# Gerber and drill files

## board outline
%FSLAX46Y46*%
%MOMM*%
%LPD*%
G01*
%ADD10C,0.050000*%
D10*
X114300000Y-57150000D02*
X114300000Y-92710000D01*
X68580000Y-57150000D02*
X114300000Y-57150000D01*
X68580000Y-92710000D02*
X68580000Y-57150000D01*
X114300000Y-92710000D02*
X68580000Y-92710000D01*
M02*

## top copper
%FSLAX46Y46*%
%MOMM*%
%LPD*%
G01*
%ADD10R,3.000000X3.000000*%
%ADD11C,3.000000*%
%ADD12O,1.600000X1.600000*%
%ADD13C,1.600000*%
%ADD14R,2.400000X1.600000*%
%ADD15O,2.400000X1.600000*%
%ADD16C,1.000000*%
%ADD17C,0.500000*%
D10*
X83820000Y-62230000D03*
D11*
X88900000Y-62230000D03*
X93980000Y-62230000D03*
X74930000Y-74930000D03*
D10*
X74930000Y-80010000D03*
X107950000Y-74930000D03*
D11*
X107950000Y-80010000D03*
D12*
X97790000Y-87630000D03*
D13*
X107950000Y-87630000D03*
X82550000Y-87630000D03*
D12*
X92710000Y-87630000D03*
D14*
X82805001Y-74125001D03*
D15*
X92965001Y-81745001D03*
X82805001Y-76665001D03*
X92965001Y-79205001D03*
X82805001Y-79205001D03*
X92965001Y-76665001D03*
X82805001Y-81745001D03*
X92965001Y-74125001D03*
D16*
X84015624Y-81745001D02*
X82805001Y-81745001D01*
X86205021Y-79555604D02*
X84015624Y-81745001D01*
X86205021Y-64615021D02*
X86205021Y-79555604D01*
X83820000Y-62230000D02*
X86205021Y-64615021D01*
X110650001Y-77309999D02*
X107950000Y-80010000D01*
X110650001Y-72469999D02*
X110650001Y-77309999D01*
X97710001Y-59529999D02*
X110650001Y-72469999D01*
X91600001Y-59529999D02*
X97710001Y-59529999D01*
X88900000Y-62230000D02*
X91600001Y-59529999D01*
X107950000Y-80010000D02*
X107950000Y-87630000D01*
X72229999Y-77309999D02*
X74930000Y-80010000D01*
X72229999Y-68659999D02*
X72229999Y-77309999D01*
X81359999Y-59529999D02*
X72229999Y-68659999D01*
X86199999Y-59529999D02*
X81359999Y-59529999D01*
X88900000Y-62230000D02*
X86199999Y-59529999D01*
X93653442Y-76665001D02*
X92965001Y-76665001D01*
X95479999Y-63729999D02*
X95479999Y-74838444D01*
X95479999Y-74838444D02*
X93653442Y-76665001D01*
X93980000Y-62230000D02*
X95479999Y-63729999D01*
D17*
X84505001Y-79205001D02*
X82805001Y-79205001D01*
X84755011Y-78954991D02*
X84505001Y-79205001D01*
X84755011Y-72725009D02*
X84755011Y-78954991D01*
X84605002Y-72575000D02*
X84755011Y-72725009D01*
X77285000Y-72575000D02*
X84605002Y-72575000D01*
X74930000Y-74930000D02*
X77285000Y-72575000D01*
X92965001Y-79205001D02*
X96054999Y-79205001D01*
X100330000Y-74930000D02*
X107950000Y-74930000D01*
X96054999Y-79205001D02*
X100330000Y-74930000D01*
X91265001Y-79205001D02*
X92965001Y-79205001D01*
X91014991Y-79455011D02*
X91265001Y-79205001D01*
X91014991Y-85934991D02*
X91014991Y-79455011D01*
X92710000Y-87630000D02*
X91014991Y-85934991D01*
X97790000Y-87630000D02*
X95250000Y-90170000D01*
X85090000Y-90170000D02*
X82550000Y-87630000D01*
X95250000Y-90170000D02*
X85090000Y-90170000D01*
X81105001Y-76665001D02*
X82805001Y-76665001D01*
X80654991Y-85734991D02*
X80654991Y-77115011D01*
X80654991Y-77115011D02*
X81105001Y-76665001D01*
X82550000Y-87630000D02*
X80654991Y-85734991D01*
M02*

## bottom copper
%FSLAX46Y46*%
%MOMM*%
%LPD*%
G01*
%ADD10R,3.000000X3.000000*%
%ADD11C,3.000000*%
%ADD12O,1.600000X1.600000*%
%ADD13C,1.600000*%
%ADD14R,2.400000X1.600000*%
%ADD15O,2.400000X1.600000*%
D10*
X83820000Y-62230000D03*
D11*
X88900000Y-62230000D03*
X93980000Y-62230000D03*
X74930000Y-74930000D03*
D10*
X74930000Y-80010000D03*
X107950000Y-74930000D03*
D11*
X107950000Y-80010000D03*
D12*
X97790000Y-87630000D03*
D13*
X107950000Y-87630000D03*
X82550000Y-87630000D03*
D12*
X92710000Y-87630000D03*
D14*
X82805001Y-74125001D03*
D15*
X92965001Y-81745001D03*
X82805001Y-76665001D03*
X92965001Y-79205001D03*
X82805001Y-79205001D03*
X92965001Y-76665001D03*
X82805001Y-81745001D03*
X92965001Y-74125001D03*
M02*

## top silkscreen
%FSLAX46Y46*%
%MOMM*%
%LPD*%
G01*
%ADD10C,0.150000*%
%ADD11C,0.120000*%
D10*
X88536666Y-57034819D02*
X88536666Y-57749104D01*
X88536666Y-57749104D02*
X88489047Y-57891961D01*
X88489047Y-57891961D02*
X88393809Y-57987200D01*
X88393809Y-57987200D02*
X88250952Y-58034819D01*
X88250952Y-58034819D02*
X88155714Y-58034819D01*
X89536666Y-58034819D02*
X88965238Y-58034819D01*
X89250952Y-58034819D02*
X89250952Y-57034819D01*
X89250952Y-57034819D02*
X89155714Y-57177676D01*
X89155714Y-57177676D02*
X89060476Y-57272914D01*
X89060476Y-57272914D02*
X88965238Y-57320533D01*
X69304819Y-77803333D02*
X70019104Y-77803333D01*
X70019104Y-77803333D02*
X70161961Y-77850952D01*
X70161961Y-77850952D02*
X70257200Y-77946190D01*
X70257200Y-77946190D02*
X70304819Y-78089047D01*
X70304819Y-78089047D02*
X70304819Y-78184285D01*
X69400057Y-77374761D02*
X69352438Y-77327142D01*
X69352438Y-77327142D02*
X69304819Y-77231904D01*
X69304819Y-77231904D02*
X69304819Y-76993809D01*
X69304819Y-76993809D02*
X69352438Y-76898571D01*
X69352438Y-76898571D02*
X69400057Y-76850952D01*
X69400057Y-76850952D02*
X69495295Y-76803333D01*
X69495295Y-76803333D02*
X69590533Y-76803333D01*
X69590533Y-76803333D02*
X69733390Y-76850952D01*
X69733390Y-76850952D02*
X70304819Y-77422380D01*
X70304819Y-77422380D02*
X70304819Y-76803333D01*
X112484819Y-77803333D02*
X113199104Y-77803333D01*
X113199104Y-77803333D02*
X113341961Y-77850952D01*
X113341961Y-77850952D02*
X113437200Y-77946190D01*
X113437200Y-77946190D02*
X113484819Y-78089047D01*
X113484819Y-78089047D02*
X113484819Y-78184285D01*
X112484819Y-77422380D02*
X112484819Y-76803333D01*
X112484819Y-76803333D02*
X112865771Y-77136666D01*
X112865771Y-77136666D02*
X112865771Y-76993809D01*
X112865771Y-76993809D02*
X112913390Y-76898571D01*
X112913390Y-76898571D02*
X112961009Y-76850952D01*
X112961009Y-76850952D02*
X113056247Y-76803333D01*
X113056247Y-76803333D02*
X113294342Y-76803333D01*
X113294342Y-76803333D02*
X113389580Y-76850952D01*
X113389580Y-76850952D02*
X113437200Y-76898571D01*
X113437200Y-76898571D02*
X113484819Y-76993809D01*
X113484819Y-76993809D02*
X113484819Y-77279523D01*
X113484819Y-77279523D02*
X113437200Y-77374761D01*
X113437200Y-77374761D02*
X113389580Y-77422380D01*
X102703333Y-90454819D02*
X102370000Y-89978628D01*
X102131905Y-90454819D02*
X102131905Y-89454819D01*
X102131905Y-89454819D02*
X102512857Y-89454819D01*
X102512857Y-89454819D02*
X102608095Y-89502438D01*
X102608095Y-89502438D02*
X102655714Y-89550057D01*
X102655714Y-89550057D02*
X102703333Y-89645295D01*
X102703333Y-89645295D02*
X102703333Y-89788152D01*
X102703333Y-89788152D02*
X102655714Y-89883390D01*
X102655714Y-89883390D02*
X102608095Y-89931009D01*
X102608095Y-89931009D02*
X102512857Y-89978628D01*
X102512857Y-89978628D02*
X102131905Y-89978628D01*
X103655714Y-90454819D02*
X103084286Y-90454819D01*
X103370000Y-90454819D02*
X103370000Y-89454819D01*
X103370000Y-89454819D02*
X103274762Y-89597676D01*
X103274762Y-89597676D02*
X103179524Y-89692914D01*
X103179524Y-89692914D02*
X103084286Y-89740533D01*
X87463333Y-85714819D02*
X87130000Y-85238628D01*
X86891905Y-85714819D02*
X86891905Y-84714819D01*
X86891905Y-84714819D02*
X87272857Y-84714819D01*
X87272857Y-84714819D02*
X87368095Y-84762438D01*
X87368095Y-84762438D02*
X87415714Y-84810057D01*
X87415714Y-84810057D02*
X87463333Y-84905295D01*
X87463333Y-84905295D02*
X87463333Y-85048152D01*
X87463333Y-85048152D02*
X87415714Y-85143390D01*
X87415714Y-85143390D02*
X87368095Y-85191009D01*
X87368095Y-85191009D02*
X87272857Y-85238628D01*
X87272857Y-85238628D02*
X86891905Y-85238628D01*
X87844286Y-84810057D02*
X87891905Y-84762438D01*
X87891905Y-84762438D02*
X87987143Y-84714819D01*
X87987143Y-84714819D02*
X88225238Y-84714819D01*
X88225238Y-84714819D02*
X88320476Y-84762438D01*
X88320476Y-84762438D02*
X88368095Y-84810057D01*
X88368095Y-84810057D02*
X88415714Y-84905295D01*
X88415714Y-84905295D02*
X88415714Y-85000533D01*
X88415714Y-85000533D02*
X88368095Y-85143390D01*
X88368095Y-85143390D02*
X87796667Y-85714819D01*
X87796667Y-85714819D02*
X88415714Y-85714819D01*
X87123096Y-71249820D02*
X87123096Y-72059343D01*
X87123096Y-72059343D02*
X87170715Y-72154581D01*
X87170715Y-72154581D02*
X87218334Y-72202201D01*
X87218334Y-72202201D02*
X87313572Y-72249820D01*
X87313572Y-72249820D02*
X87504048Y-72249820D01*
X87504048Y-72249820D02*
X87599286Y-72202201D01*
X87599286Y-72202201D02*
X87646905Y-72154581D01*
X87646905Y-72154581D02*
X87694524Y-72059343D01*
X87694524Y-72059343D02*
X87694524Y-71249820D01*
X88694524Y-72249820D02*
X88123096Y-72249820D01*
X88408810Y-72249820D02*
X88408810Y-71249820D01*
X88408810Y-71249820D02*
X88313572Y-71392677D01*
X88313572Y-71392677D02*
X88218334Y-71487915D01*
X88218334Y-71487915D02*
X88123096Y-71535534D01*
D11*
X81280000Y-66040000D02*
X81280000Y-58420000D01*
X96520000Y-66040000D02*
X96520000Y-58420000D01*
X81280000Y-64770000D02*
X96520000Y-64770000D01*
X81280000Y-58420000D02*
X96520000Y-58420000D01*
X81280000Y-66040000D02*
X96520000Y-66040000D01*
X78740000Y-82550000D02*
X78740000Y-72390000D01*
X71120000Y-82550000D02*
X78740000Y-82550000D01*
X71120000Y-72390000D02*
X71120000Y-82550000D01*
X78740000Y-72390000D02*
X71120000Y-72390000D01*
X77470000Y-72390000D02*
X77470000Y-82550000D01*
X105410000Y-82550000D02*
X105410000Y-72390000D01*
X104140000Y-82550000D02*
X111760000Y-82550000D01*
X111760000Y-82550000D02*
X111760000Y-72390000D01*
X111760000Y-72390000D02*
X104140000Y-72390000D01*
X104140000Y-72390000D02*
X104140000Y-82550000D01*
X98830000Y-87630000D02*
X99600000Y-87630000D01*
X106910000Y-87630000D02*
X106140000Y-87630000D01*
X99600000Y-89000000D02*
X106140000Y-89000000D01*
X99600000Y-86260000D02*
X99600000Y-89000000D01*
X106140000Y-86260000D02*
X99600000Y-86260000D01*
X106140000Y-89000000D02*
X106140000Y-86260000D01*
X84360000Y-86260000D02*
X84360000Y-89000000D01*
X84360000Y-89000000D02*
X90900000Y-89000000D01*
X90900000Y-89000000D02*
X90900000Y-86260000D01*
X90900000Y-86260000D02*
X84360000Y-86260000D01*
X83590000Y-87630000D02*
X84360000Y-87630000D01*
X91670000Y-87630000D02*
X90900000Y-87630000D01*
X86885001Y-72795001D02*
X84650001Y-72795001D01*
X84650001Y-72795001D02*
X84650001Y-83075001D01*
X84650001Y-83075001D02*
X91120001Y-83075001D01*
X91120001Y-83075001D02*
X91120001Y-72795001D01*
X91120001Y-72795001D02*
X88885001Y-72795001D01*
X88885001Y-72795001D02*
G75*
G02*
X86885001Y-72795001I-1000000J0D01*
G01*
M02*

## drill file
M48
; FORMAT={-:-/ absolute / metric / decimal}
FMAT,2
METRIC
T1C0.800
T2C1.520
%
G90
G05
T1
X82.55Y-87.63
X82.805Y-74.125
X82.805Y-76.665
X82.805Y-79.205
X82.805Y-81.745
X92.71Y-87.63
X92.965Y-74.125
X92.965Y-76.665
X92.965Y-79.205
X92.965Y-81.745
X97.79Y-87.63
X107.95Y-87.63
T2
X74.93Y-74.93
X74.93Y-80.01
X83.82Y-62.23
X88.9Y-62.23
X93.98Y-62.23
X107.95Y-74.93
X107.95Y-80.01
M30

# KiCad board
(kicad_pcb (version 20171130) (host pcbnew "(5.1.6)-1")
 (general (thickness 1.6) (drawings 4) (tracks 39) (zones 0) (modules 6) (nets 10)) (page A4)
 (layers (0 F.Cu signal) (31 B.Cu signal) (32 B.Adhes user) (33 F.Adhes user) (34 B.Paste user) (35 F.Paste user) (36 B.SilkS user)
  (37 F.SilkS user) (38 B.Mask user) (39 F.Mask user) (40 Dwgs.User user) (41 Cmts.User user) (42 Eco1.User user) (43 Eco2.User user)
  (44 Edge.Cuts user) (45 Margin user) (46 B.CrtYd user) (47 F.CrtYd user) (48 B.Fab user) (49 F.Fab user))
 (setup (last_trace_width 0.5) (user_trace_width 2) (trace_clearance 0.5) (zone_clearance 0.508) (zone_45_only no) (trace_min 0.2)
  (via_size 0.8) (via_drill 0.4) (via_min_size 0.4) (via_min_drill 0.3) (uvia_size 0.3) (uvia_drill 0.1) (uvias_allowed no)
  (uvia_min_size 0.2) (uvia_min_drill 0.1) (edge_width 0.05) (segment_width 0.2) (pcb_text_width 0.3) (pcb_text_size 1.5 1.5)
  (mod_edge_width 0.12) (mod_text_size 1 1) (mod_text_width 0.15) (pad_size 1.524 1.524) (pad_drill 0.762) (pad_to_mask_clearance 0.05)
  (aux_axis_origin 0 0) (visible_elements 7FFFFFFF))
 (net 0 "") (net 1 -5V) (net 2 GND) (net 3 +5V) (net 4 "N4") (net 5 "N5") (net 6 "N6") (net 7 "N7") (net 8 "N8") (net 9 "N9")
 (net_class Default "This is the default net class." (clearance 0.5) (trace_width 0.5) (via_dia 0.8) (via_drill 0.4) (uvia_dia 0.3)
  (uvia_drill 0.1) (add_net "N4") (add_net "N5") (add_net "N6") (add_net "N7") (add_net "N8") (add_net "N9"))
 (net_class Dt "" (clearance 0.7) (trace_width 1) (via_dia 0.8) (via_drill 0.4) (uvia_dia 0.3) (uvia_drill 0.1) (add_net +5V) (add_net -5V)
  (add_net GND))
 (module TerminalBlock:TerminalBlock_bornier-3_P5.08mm (layer F.Cu) (at 83.82 62.23)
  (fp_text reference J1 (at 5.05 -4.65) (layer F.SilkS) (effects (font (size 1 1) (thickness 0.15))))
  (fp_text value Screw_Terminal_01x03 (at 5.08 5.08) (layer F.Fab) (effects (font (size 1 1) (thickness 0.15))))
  (fp_line (start -2.54 3.81) (end -2.54 -3.81) (layer F.SilkS) (width 0.12))
  (fp_line (start 12.7 3.81) (end 12.7 -3.81) (layer F.SilkS) (width 0.12))
  (fp_line (start -2.54 2.54) (end 12.7 2.54) (layer F.SilkS) (width 0.12))
  (fp_line (start -2.54 -3.81) (end 12.7 -3.81) (layer F.SilkS) (width 0.12))
  (fp_line (start -2.54 3.81) (end 12.7 3.81) (layer F.SilkS) (width 0.12))
  (pad 1 thru_hole rect (at 0 0) (size 3 3) (drill 1.52) (layers *.Cu *.Mask) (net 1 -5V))
  (pad 2 thru_hole circle (at 5.08 0) (size 3 3) (drill 1.52) (layers *.Cu *.Mask) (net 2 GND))
  (pad 3 thru_hole circle (at 10.16 0) (size 3 3) (drill 1.52) (layers *.Cu *.Mask) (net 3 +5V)))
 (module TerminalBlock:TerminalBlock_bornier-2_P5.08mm (layer F.Cu) (at 74.93 80.01 90)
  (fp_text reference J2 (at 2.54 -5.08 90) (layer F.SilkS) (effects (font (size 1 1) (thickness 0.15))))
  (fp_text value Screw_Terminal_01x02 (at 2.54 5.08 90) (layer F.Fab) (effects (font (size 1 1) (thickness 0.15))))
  (fp_line (start -2.54 3.81) (end 7.62 3.81) (layer F.SilkS) (width 0.12))
  (fp_line (start -2.54 -3.81) (end -2.54 3.81) (layer F.SilkS) (width 0.12))
  (fp_line (start 7.62 -3.81) (end -2.54 -3.81) (layer F.SilkS) (width 0.12))
  (fp_line (start 7.62 3.81) (end 7.62 -3.81) (layer F.SilkS) (width 0.12))
  (fp_line (start 7.62 2.54) (end -2.54 2.54) (layer F.SilkS) (width 0.12))
  (pad 2 thru_hole circle (at 5.08 0 90) (size 3 3) (drill 1.52) (layers *.Cu *.Mask) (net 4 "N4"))
  (pad 1 thru_hole rect (at 0 0 90) (size 3 3) (drill 1.52) (layers *.Cu *.Mask) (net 2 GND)))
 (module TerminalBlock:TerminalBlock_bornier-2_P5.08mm (layer F.Cu) (at 107.95 74.93 270)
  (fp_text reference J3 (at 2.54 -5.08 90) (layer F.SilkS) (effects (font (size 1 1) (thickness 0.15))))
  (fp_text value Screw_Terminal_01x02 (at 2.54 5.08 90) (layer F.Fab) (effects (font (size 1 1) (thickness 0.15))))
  (fp_line (start 7.62 2.54) (end -2.54 2.54) (layer F.SilkS) (width 0.12))
  (fp_line (start 7.62 3.81) (end 7.62 -3.81) (layer F.SilkS) (width 0.12))
  (fp_line (start 7.62 -3.81) (end -2.54 -3.81) (layer F.SilkS) (width 0.12))
  (fp_line (start -2.54 -3.81) (end -2.54 3.81) (layer F.SilkS) (width 0.12))
  (fp_line (start -2.54 3.81) (end 7.62 3.81) (layer F.SilkS) (width 0.12))
  (pad 1 thru_hole rect (at 0 0 270) (size 3 3) (drill 1.52) (layers *.Cu *.Mask) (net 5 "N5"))
  (pad 2 thru_hole circle (at 5.08 0 270) (size 3 3) (drill 1.52) (layers *.Cu *.Mask) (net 2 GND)))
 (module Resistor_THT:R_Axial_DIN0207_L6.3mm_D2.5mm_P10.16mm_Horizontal (layer F.Cu) (at 107.95 87.63 180)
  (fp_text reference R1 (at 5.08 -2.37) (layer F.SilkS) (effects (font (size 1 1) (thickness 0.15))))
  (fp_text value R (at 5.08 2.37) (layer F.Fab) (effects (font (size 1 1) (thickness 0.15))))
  (fp_line (start 9.12 0) (end 8.35 0) (layer F.SilkS) (width 0.12))
  (fp_line (start 1.04 0) (end 1.81 0) (layer F.SilkS) (width 0.12))
  (fp_line (start 8.35 -1.37) (end 1.81 -1.37) (layer F.SilkS) (width 0.12))
  (fp_line (start 8.35 1.37) (end 8.35 -1.37) (layer F.SilkS) (width 0.12))
  (fp_line (start 1.81 1.37) (end 8.35 1.37) (layer F.SilkS) (width 0.12))
  (fp_line (start 1.81 -1.37) (end 1.81 1.37) (layer F.SilkS) (width 0.12))
  (pad 2 thru_hole oval (at 10.16 0 180) (size 1.6 1.6) (drill 0.8) (layers *.Cu *.Mask) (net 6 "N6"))
  (pad 1 thru_hole circle (at 0 0 180) (size 1.6 1.6) (drill 0.8) (layers *.Cu *.Mask) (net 2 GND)))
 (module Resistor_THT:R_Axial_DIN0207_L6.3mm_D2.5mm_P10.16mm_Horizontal (layer F.Cu) (at 82.55 87.63)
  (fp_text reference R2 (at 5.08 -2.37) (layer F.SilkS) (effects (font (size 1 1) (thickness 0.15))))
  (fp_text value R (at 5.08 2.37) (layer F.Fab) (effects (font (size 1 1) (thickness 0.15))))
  (fp_line (start 1.81 -1.37) (end 1.81 1.37) (layer F.SilkS) (width 0.12))
  (fp_line (start 1.81 1.37) (end 8.35 1.37) (layer F.SilkS) (width 0.12))
  (fp_line (start 8.35 1.37) (end 8.35 -1.37) (layer F.SilkS) (width 0.12))
  (fp_line (start 8.35 -1.37) (end 1.81 -1.37) (layer F.SilkS) (width 0.12))
  (fp_line (start 1.04 0) (end 1.81 0) (layer F.SilkS) (width 0.12))
  (fp_line (start 9.12 0) (end 8.35 0) (layer F.SilkS) (width 0.12))
  (pad 1 thru_hole circle (at 0 0) (size 1.6 1.6) (drill 0.8) (layers *.Cu *.Mask) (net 6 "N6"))
  (pad 2 thru_hole oval (at 10.16 0) (size 1.6 1.6) (drill 0.8) (layers *.Cu *.Mask) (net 5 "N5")))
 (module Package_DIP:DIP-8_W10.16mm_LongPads (layer F.Cu) (at 82.805001 74.125001)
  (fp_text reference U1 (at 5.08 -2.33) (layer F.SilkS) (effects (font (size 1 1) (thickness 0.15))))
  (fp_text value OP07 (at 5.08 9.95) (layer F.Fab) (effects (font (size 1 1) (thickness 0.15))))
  (fp_line (start 4.08 -1.33) (end 1.845 -1.33) (layer F.SilkS) (width 0.12))
  (fp_line (start 1.845 -1.33) (end 1.845 8.95) (layer F.SilkS) (width 0.12))
  (fp_line (start 1.845 8.95) (end 8.315 8.95) (layer F.SilkS) (width 0.12))
  (fp_line (start 8.315 8.95) (end 8.315 -1.33) (layer F.SilkS) (width 0.12))
  (fp_line (start 8.315 -1.33) (end 6.08 -1.33) (layer F.SilkS) (width 0.12))
  (fp_arc (start 5.08 -1.33) (end 4.08 -1.33) (angle -180) (layer F.SilkS) (width 0.12))
  (pad 1 thru_hole rect (at 0 0) (size 2.4 1.6) (drill 0.8) (layers *.Cu *.Mask) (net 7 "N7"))
  (pad 5 thru_hole oval (at 10.16 7.62) (size 2.4 1.6) (drill 0.8) (layers *.Cu *.Mask) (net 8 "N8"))
  (pad 2 thru_hole oval (at 0 2.54) (size 2.4 1.6) (drill 0.8) (layers *.Cu *.Mask) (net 6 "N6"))
  (pad 6 thru_hole oval (at 10.16 5.08) (size 2.4 1.6) (drill 0.8) (layers *.Cu *.Mask) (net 5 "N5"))
  (pad 3 thru_hole oval (at 0 5.08) (size 2.4 1.6) (drill 0.8) (layers *.Cu *.Mask) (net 4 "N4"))
  (pad 7 thru_hole oval (at 10.16 2.54) (size 2.4 1.6) (drill 0.8) (layers *.Cu *.Mask) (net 3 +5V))
  (pad 4 thru_hole oval (at 0 7.62) (size 2.4 1.6) (drill 0.8) (layers *.Cu *.Mask) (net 1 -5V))
  (pad 8 thru_hole oval (at 10.16 0) (size 2.4 1.6) (drill 0.8) (layers *.Cu *.Mask) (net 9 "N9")))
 (gr_line (start 114.3 57.15) (end 114.3 92.71) (layer Edge.Cuts) (width 0.05))
 (gr_line (start 68.58 57.15) (end 114.3 57.15) (layer Edge.Cuts) (width 0.05))
 (gr_line (start 68.58 92.71) (end 68.58 57.15) (layer Edge.Cuts) (width 0.05))
 (gr_line (start 114.3 92.71) (end 68.58 92.71) (layer Edge.Cuts) (width 0.05))
 (segment (start 84.015624 81.745001) (end 82.805001 81.745001) (width 1) (layer F.Cu) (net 1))
 (segment (start 86.205021 79.555604) (end 84.015624 81.745001) (width 1) (layer F.Cu) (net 1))
 (segment (start 86.205021 64.615021) (end 86.205021 79.555604) (width 1) (layer F.Cu) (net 1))
 (segment (start 83.82 62.23) (end 86.205021 64.615021) (width 1) (layer F.Cu) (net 1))
 (segment (start 110.650001 77.309999) (end 107.95 80.01) (width 1) (layer F.Cu) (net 2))
 (segment (start 110.650001 72.469999) (end 110.650001 77.309999) (width 1) (layer F.Cu) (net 2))
 (segment (start 97.710001 59.529999) (end 110.650001 72.469999) (width 1) (layer F.Cu) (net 2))
 (segment (start 91.600001 59.529999) (end 97.710001 59.529999) (width 1) (layer F.Cu) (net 2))
 (segment (start 88.9 62.23) (end 91.600001 59.529999) (width 1) (layer F.Cu) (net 2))
 (segment (start 107.95 80.01) (end 107.95 87.63) (width 1) (layer F.Cu) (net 2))
 (segment (start 72.229999 77.309999) (end 74.93 80.01) (width 1) (layer F.Cu) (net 2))
 (segment (start 72.229999 68.659999) (end 72.229999 77.309999) (width 1) (layer F.Cu) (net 2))
 (segment (start 81.359999 59.529999) (end 72.229999 68.659999) (width 1) (layer F.Cu) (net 2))
 (segment (start 86.199999 59.529999) (end 81.359999 59.529999) (width 1) (layer F.Cu) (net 2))
 (segment (start 88.9 62.23) (end 86.199999 59.529999) (width 1) (layer F.Cu) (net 2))
 (segment (start 93.653442 76.665001) (end 92.965001 76.665001) (width 1) (layer F.Cu) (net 3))
 (segment (start 95.479999 63.729999) (end 95.479999 74.838444) (width 1) (layer F.Cu) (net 3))
 (segment (start 95.479999 74.838444) (end 93.653442 76.665001) (width 1) (layer F.Cu) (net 3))
 (segment (start 93.98 62.23) (end 95.479999 63.729999) (width 1) (layer F.Cu) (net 3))
 (segment (start 84.505001 79.205001) (end 82.805001 79.205001) (width 0.5) (layer F.Cu) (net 4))
 (segment (start 84.755011 78.954991) (end 84.505001 79.205001) (width 0.5) (layer F.Cu) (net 4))
 (segment (start 84.755011 72.725009) (end 84.755011 78.954991) (width 0.5) (layer F.Cu) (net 4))
 (segment (start 84.605002 72.575) (end 84.755011 72.725009) (width 0.5) (layer F.Cu) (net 4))
 (segment (start 77.285 72.575) (end 84.605002 72.575) (width 0.5) (layer F.Cu) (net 4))
 (segment (start 74.93 74.93) (end 77.285 72.575) (width 0.5) (layer F.Cu) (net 4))
 (segment (start 92.965001 79.205001) (end 96.054999 79.205001) (width 0.5) (layer F.Cu) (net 5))
 (segment (start 100.33 74.93) (end 107.95 74.93) (width 0.5) (layer F.Cu) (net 5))
 (segment (start 96.054999 79.205001) (end 100.33 74.93) (width 0.5) (layer F.Cu) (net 5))
 (segment (start 91.265001 79.205001) (end 92.965001 79.205001) (width 0.5) (layer F.Cu) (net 5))
 (segment (start 91.014991 79.455011) (end 91.265001 79.205001) (width 0.5) (layer F.Cu) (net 5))
 (segment (start 91.014991 85.934991) (end 91.014991 79.455011) (width 0.5) (layer F.Cu) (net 5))
 (segment (start 92.71 87.63) (end 91.014991 85.934991) (width 0.5) (layer F.Cu) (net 5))
 (segment (start 97.79 87.63) (end 95.25 90.17) (width 0.5) (layer F.Cu) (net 6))
 (segment (start 85.09 90.17) (end 82.55 87.63) (width 0.5) (layer F.Cu) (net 6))
 (segment (start 95.25 90.17) (end 85.09 90.17) (width 0.5) (layer F.Cu) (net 6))
 (segment (start 81.105001 76.665001) (end 82.805001 76.665001) (width 0.5) (layer F.Cu) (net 6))
 (segment (start 80.654991 85.734991) (end 80.654991 77.115011) (width 0.5) (layer F.Cu) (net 6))
 (segment (start 80.654991 77.115011) (end 81.105001 76.665001) (width 0.5) (layer F.Cu) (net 6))
 (segment (start 82.55 87.63) (end 80.654991 85.734991) (width 0.5) (layer F.Cu) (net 6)))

